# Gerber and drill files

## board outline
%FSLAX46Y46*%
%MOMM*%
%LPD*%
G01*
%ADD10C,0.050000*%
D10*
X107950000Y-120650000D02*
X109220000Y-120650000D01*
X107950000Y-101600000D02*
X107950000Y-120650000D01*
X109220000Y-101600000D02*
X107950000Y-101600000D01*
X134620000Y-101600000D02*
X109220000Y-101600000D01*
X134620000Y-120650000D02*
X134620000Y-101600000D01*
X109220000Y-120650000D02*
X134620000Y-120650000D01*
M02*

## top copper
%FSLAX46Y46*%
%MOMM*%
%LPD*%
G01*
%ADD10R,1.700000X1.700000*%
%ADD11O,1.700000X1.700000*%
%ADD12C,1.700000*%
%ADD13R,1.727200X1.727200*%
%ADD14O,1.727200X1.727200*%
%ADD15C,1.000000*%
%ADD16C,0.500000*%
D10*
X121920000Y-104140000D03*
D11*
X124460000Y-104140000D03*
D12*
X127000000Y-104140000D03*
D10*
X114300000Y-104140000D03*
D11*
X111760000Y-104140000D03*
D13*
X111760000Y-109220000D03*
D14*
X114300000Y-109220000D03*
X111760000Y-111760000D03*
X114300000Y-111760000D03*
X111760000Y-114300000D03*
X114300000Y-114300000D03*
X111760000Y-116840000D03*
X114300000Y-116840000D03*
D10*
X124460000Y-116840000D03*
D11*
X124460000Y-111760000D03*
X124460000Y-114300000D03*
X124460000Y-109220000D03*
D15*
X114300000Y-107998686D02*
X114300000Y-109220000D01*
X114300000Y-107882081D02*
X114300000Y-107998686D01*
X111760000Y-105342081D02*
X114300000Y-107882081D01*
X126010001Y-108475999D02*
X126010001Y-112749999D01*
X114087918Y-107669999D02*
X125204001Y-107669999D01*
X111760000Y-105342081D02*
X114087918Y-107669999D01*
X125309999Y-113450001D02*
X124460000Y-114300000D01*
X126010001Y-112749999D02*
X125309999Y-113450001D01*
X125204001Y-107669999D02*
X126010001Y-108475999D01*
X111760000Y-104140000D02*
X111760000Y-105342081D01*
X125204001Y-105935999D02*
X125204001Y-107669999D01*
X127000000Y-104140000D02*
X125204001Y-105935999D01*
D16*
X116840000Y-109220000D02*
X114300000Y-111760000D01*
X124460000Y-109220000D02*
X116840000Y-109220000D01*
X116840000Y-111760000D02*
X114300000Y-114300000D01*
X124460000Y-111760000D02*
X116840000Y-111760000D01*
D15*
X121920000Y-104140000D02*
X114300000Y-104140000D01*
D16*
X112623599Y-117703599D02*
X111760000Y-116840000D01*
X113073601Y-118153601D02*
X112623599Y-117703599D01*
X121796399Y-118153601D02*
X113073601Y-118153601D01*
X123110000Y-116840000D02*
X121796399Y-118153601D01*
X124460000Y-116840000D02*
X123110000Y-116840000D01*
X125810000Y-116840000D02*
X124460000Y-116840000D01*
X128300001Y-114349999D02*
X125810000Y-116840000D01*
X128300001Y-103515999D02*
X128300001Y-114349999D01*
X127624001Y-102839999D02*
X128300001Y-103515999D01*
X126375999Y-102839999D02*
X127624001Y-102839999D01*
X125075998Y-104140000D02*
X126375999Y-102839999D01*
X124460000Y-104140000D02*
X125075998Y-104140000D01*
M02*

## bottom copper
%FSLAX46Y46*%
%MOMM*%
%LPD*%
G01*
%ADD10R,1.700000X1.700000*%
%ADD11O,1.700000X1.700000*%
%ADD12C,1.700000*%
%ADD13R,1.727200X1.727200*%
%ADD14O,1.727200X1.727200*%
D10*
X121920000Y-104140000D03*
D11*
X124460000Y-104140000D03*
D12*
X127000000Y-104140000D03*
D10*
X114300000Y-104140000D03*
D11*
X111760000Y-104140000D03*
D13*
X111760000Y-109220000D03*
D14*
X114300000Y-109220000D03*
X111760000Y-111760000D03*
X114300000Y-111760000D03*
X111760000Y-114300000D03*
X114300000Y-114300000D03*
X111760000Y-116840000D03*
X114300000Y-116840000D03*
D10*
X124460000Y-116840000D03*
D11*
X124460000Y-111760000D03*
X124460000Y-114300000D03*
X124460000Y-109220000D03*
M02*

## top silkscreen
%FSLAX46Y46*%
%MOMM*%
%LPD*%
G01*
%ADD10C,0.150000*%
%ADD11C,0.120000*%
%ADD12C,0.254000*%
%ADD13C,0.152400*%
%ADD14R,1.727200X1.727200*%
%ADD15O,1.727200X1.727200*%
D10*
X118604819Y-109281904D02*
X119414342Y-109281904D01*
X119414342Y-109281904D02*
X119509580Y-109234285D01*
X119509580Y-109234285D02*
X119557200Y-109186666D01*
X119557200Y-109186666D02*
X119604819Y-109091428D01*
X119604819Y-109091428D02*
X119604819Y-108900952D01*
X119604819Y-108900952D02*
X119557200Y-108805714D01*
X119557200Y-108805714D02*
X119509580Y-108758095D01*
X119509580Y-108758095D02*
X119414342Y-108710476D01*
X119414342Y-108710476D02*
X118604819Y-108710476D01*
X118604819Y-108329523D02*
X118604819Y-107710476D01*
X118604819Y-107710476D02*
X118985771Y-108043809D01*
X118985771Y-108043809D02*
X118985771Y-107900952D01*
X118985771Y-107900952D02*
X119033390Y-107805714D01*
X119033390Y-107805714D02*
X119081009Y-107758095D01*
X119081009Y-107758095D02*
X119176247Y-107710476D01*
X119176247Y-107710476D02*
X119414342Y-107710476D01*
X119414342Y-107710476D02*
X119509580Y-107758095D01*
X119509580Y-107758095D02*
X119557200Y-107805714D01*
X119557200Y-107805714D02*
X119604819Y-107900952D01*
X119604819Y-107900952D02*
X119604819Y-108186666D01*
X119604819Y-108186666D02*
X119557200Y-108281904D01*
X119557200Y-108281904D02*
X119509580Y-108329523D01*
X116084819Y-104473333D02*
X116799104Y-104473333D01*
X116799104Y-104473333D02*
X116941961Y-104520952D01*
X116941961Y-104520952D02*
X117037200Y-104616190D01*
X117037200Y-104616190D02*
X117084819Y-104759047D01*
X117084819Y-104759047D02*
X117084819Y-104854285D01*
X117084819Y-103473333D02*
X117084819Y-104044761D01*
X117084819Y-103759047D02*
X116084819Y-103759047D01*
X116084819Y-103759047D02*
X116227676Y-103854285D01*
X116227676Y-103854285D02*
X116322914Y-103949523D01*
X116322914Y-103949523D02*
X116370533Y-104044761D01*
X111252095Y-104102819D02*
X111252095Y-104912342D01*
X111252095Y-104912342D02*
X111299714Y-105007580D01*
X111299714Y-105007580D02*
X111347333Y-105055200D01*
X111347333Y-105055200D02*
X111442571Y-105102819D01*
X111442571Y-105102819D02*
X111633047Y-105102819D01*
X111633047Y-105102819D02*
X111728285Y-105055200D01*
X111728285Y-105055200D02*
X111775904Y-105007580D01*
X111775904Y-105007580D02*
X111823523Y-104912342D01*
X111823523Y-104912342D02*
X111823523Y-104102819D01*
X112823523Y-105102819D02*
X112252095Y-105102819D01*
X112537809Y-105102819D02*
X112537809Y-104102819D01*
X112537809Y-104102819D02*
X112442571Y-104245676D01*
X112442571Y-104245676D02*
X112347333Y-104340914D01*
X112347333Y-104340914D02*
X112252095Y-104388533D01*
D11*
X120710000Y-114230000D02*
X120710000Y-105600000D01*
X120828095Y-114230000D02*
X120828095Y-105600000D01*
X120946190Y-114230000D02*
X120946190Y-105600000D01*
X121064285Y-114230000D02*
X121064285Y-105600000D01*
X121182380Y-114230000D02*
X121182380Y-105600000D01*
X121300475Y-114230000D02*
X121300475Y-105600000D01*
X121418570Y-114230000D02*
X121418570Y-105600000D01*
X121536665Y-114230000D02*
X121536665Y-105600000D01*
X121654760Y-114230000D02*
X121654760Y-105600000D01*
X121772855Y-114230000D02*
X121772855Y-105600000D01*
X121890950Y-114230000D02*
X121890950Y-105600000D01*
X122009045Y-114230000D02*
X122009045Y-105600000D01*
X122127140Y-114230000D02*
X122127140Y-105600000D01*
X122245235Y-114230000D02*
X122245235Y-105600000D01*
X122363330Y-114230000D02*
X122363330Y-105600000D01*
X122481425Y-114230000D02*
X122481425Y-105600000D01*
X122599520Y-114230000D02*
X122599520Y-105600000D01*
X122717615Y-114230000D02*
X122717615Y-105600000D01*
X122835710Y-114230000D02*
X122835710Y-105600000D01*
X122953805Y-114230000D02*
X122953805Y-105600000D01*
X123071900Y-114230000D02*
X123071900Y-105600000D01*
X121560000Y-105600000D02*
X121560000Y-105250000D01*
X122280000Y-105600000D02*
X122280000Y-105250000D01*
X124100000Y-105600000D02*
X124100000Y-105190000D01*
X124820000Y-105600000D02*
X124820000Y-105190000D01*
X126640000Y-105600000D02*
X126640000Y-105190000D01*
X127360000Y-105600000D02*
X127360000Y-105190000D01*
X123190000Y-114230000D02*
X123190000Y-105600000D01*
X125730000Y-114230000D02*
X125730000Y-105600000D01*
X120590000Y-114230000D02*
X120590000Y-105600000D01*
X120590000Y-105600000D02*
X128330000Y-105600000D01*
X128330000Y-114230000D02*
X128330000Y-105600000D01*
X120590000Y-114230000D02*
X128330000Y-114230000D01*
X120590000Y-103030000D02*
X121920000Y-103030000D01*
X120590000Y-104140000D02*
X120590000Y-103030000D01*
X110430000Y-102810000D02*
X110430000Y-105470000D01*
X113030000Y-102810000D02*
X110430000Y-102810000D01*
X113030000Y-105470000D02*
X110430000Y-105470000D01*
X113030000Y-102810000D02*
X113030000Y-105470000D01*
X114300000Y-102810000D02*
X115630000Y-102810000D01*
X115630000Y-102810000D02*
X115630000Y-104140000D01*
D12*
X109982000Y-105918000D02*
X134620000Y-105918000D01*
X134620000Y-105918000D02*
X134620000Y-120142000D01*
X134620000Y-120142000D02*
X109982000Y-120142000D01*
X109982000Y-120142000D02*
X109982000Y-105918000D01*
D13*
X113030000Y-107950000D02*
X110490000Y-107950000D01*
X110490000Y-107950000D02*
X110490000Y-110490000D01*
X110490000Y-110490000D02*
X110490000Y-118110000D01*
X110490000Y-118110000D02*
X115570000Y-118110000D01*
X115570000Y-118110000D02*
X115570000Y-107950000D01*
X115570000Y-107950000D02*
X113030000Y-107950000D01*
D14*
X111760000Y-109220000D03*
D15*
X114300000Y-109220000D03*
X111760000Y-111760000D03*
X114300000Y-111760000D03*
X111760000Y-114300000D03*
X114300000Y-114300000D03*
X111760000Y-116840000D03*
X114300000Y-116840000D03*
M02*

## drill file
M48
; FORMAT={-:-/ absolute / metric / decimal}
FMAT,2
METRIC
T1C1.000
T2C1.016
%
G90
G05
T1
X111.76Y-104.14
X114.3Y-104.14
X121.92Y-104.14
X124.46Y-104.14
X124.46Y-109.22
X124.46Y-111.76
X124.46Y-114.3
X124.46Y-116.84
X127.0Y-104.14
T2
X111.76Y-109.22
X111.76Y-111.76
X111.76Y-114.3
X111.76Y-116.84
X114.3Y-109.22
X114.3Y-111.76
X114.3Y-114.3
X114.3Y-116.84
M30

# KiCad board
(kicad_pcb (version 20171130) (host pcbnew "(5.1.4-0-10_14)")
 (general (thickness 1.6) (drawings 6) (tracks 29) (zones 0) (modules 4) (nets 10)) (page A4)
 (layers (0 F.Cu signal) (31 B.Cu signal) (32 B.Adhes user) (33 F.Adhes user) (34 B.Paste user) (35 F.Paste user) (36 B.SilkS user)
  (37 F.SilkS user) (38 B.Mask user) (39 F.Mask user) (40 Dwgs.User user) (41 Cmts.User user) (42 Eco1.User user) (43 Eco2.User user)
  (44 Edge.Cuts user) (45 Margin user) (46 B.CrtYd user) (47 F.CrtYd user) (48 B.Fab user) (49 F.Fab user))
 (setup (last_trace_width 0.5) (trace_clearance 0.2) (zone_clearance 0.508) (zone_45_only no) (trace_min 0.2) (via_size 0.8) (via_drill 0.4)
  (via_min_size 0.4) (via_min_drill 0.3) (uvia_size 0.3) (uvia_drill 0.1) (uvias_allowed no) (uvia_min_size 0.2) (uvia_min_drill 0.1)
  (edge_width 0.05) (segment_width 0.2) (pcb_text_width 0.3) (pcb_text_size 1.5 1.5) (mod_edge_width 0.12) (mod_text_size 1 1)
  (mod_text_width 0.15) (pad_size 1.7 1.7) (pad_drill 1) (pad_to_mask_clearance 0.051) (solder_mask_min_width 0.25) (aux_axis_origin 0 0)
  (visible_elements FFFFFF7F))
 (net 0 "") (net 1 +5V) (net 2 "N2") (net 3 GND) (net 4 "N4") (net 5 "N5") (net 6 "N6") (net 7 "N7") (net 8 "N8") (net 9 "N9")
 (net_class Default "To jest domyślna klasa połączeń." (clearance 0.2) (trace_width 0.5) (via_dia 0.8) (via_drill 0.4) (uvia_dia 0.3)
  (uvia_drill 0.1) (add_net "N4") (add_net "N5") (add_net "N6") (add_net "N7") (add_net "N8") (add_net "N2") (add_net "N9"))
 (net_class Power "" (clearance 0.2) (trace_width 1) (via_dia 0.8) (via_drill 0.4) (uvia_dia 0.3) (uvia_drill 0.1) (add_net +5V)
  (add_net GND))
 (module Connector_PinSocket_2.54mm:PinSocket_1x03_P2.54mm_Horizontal (layer F.Cu) (at 121.92 104.14 90)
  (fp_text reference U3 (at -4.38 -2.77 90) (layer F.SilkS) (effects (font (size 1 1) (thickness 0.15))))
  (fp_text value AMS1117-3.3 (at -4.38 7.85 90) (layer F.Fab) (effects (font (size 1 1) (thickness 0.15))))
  (fp_line (start -10.09 -1.21) (end -1.46 -1.21) (layer F.SilkS) (width 0.12))
  (fp_line (start -10.09 -1.091905) (end -1.46 -1.091905) (layer F.SilkS) (width 0.12))
  (fp_line (start -10.09 -0.97381) (end -1.46 -0.97381) (layer F.SilkS) (width 0.12))
  (fp_line (start -10.09 -0.855715) (end -1.46 -0.855715) (layer F.SilkS) (width 0.12))
  (fp_line (start -10.09 -0.73762) (end -1.46 -0.73762) (layer F.SilkS) (width 0.12))
  (fp_line (start -10.09 -0.619525) (end -1.46 -0.619525) (layer F.SilkS) (width 0.12))
  (fp_line (start -10.09 -0.50143) (end -1.46 -0.50143) (layer F.SilkS) (width 0.12))
  (fp_line (start -10.09 -0.383335) (end -1.46 -0.383335) (layer F.SilkS) (width 0.12))
  (fp_line (start -10.09 -0.26524) (end -1.46 -0.26524) (layer F.SilkS) (width 0.12))
  (fp_line (start -10.09 -0.147145) (end -1.46 -0.147145) (layer F.SilkS) (width 0.12))
  (fp_line (start -10.09 -0.02905) (end -1.46 -0.02905) (layer F.SilkS) (width 0.12))
  (fp_line (start -10.09 0.089045) (end -1.46 0.089045) (layer F.SilkS) (width 0.12))
  (fp_line (start -10.09 0.20714) (end -1.46 0.20714) (layer F.SilkS) (width 0.12))
  (fp_line (start -10.09 0.325235) (end -1.46 0.325235) (layer F.SilkS) (width 0.12))
  (fp_line (start -10.09 0.44333) (end -1.46 0.44333) (layer F.SilkS) (width 0.12))
  (fp_line (start -10.09 0.561425) (end -1.46 0.561425) (layer F.SilkS) (width 0.12))
  (fp_line (start -10.09 0.67952) (end -1.46 0.67952) (layer F.SilkS) (width 0.12))
  (fp_line (start -10.09 0.797615) (end -1.46 0.797615) (layer F.SilkS) (width 0.12))
  (fp_line (start -10.09 0.91571) (end -1.46 0.91571) (layer F.SilkS) (width 0.12))
  (fp_line (start -10.09 1.033805) (end -1.46 1.033805) (layer F.SilkS) (width 0.12))
  (fp_line (start -10.09 1.1519) (end -1.46 1.1519) (layer F.SilkS) (width 0.12))
  (fp_line (start -1.46 -0.36) (end -1.11 -0.36) (layer F.SilkS) (width 0.12))
  (fp_line (start -1.46 0.36) (end -1.11 0.36) (layer F.SilkS) (width 0.12))
  (fp_line (start -1.46 2.18) (end -1.05 2.18) (layer F.SilkS) (width 0.12))
  (fp_line (start -1.46 2.9) (end -1.05 2.9) (layer F.SilkS) (width 0.12))
  (fp_line (start -1.46 4.72) (end -1.05 4.72) (layer F.SilkS) (width 0.12))
  (fp_line (start -1.46 5.44) (end -1.05 5.44) (layer F.SilkS) (width 0.12))
  (fp_line (start -10.09 1.27) (end -1.46 1.27) (layer F.SilkS) (width 0.12))
  (fp_line (start -10.09 3.81) (end -1.46 3.81) (layer F.SilkS) (width 0.12))
  (fp_line (start -10.09 -1.33) (end -1.46 -1.33) (layer F.SilkS) (width 0.12))
  (fp_line (start -1.46 -1.33) (end -1.46 6.41) (layer F.SilkS) (width 0.12))
  (fp_line (start -10.09 6.41) (end -1.46 6.41) (layer F.SilkS) (width 0.12))
  (fp_line (start -10.09 -1.33) (end -10.09 6.41) (layer F.SilkS) (width 0.12))
  (fp_line (start 1.11 -1.33) (end 1.11 0) (layer F.SilkS) (width 0.12))
  (fp_line (start 0 -1.33) (end 1.11 -1.33) (layer F.SilkS) (width 0.12))
  (pad 3 thru_hole rect (at 0 0 90) (size 1.7 1.7) (drill 1) (layers *.Cu *.Mask) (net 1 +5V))
  (pad 2 thru_hole oval (at 0 2.54 90) (size 1.7 1.7) (drill 1) (layers *.Cu *.Mask) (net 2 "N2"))
  (pad 1 thru_hole circle (at 0 5.08 90) (size 1.7 1.7) (drill 1) (layers *.Cu *.Mask) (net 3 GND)))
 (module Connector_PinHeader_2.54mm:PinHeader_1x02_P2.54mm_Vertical (layer F.Cu) (at 114.3 104.14 270)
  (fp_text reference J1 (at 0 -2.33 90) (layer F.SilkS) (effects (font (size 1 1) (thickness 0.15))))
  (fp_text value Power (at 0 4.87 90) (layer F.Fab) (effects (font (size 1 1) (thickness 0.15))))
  (fp_line (start -1.33 3.87) (end 1.33 3.87) (layer F.SilkS) (width 0.12))
  (fp_line (start -1.33 1.27) (end -1.33 3.87) (layer F.SilkS) (width 0.12))
  (fp_line (start 1.33 1.27) (end 1.33 3.87) (layer F.SilkS) (width 0.12))
  (fp_line (start -1.33 1.27) (end 1.33 1.27) (layer F.SilkS) (width 0.12))
  (fp_line (start -1.33 0) (end -1.33 -1.33) (layer F.SilkS) (width 0.12))
  (fp_line (start -1.33 -1.33) (end 0 -1.33) (layer F.SilkS) (width 0.12))
  (pad 1 thru_hole rect (at 0 0 270) (size 1.7 1.7) (drill 1) (layers *.Cu *.Mask) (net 1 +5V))
  (pad 2 thru_hole oval (at 0 2.54 270) (size 1.7 1.7) (drill 1) (layers *.Cu *.Mask) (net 3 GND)))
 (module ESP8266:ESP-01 (layer F.Cu) (at 111.76 109.22)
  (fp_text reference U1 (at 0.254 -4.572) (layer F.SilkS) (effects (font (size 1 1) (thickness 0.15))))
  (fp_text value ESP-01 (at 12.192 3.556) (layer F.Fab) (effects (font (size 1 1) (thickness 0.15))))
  (fp_line (start -1.778 -3.302) (end 22.86 -3.302) (layer F.SilkS) (width 0.254))
  (fp_line (start 22.86 -3.302) (end 22.86 10.922) (layer F.SilkS) (width 0.254))
  (fp_line (start 22.86 10.922) (end -1.778 10.922) (layer F.SilkS) (width 0.254))
  (fp_line (start -1.778 10.922) (end -1.778 -3.302) (layer F.SilkS) (width 0.254))
  (fp_line (start 1.27 -1.27) (end -1.27 -1.27) (layer F.SilkS) (width 0.1524))
  (fp_line (start -1.27 -1.27) (end -1.27 1.27) (layer F.SilkS) (width 0.1524))
  (fp_line (start -1.27 1.27) (end -1.27 8.89) (layer F.SilkS) (width 0.1524))
  (fp_line (start -1.27 8.89) (end 3.81 8.89) (layer F.SilkS) (width 0.1524))
  (fp_line (start 3.81 8.89) (end 3.81 -1.27) (layer F.SilkS) (width 0.1524))
  (fp_line (start 3.81 -1.27) (end 1.27 -1.27) (layer F.SilkS) (width 0.1524))
  (pad 1 thru_hole rect (at 0 0) (size 1.7272 1.7272) (drill 1.016) (layers *.Cu *.Mask F.SilkS) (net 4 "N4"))
  (pad 2 thru_hole oval (at 2.54 0) (size 1.7272 1.7272) (drill 1.016) (layers *.Cu *.Mask F.SilkS) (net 3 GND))
  (pad 3 thru_hole oval (at 0 2.54) (size 1.7272 1.7272) (drill 1.016) (layers *.Cu *.Mask F.SilkS) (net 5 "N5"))
  (pad 4 thru_hole oval (at 2.54 2.54) (size 1.7272 1.7272) (drill 1.016) (layers *.Cu *.Mask F.SilkS) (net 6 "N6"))
  (pad 5 thru_hole oval (at 0 5.08) (size 1.7272 1.7272) (drill 1.016) (layers *.Cu *.Mask F.SilkS) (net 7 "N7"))
  (pad 6 thru_hole oval (at 2.54 5.08) (size 1.7272 1.7272) (drill 1.016) (layers *.Cu *.Mask F.SilkS) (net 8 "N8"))
  (pad 7 thru_hole oval (at 0 7.62) (size 1.7272 1.7272) (drill 1.016) (layers *.Cu *.Mask F.SilkS) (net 2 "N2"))
  (pad 8 thru_hole oval (at 2.54 7.62) (size 1.7272 1.7272) (drill 1.016) (layers *.Cu *.Mask F.SilkS) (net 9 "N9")))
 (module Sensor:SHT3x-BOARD (layer B.Cu) (at 124.46 109.22 180)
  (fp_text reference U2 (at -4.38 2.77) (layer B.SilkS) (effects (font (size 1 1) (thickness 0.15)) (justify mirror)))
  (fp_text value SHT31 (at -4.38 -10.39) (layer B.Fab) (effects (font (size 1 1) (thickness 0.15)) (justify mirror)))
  (pad 5 thru_hole rect (at 0 -7.62 180) (size 1.7 1.7) (drill 1) (layers *.Cu *.Mask) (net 2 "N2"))
  (pad 4 thru_hole oval (at 0 -2.54 180) (size 1.7 1.7) (drill 1) (layers *.Cu *.Mask) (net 8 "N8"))
  (pad 8 thru_hole oval (at 0 -5.08 180) (size 1.7 1.7) (drill 1) (layers *.Cu *.Mask) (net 3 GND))
  (pad 1 thru_hole oval (at 0 0 180) (size 1.7 1.7) (drill 1) (layers *.Cu *.Mask) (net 6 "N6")))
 (gr_line (start 107.95 120.65) (end 109.22 120.65) (layer Edge.Cuts) (width 0.05))
 (gr_line (start 107.95 101.6) (end 107.95 120.65) (layer Edge.Cuts) (width 0.05))
 (gr_line (start 109.22 101.6) (end 107.95 101.6) (layer Edge.Cuts) (width 0.05))
 (gr_line (start 134.62 101.6) (end 109.22 101.6) (layer Edge.Cuts) (width 0.05))
 (gr_line (start 134.62 120.65) (end 134.62 101.6) (layer Edge.Cuts) (width 0.05))
 (gr_line (start 109.22 120.65) (end 134.62 120.65) (layer Edge.Cuts) (width 0.05))
 (segment (start 114.3 107.998686) (end 114.3 109.22) (width 1) (layer F.Cu) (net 3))
 (segment (start 114.3 107.882081) (end 114.3 107.998686) (width 1) (layer F.Cu) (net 3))
 (segment (start 111.76 105.342081) (end 114.3 107.882081) (width 1) (layer F.Cu) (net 3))
 (segment (start 126.010001 108.475999) (end 126.010001 112.749999) (width 1) (layer F.Cu) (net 3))
 (segment (start 114.087918 107.669999) (end 125.204001 107.669999) (width 1) (layer F.Cu) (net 3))
 (segment (start 111.76 105.342081) (end 114.087918 107.669999) (width 1) (layer F.Cu) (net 3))
 (segment (start 125.309999 113.450001) (end 124.46 114.3) (width 1) (layer F.Cu) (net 3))
 (segment (start 126.010001 112.749999) (end 125.309999 113.450001) (width 1) (layer F.Cu) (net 3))
 (segment (start 125.204001 107.669999) (end 126.010001 108.475999) (width 1) (layer F.Cu) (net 3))
 (segment (start 111.76 104.14) (end 111.76 105.342081) (width 1) (layer F.Cu) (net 3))
 (segment (start 125.204001 105.935999) (end 125.204001 107.669999) (width 1) (layer F.Cu) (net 3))
 (segment (start 127 104.14) (end 125.204001 105.935999) (width 1) (layer F.Cu) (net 3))
 (segment (start 116.84 109.22) (end 114.3 111.76) (width 0.5) (layer F.Cu) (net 6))
 (segment (start 124.46 109.22) (end 116.84 109.22) (width 0.5) (layer F.Cu) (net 6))
 (segment (start 116.84 111.76) (end 114.3 114.3) (width 0.5) (layer F.Cu) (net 8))
 (segment (start 124.46 111.76) (end 116.84 111.76) (width 0.5) (layer F.Cu) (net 8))
 (segment (start 121.92 104.14) (end 114.3 104.14) (width 1) (layer F.Cu) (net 1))
 (segment (start 112.623599 117.703599) (end 111.76 116.84) (width 0.5) (layer F.Cu) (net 2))
 (segment (start 113.073601 118.153601) (end 112.623599 117.703599) (width 0.5) (layer F.Cu) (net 2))
 (segment (start 121.796399 118.153601) (end 113.073601 118.153601) (width 0.5) (layer F.Cu) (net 2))
 (segment (start 123.11 116.84) (end 121.796399 118.153601) (width 0.5) (layer F.Cu) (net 2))
 (segment (start 124.46 116.84) (end 123.11 116.84) (width 0.5) (layer F.Cu) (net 2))
 (segment (start 125.81 116.84) (end 124.46 116.84) (width 0.5) (layer F.Cu) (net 2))
 (segment (start 128.300001 114.349999) (end 125.81 116.84) (width 0.5) (layer F.Cu) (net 2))
 (segment (start 128.300001 103.515999) (end 128.300001 114.349999) (width 0.5) (layer F.Cu) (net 2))
 (segment (start 127.624001 102.839999) (end 128.300001 103.515999) (width 0.5) (layer F.Cu) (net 2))
 (segment (start 126.375999 102.839999) (end 127.624001 102.839999) (width 0.5) (layer F.Cu) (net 2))
 (segment (start 125.075998 104.14) (end 126.375999 102.839999) (width 0.5) (layer F.Cu) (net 2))
 (segment (start 124.46 104.14) (end 125.075998 104.14) (width 0.5) (layer F.Cu) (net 2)))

